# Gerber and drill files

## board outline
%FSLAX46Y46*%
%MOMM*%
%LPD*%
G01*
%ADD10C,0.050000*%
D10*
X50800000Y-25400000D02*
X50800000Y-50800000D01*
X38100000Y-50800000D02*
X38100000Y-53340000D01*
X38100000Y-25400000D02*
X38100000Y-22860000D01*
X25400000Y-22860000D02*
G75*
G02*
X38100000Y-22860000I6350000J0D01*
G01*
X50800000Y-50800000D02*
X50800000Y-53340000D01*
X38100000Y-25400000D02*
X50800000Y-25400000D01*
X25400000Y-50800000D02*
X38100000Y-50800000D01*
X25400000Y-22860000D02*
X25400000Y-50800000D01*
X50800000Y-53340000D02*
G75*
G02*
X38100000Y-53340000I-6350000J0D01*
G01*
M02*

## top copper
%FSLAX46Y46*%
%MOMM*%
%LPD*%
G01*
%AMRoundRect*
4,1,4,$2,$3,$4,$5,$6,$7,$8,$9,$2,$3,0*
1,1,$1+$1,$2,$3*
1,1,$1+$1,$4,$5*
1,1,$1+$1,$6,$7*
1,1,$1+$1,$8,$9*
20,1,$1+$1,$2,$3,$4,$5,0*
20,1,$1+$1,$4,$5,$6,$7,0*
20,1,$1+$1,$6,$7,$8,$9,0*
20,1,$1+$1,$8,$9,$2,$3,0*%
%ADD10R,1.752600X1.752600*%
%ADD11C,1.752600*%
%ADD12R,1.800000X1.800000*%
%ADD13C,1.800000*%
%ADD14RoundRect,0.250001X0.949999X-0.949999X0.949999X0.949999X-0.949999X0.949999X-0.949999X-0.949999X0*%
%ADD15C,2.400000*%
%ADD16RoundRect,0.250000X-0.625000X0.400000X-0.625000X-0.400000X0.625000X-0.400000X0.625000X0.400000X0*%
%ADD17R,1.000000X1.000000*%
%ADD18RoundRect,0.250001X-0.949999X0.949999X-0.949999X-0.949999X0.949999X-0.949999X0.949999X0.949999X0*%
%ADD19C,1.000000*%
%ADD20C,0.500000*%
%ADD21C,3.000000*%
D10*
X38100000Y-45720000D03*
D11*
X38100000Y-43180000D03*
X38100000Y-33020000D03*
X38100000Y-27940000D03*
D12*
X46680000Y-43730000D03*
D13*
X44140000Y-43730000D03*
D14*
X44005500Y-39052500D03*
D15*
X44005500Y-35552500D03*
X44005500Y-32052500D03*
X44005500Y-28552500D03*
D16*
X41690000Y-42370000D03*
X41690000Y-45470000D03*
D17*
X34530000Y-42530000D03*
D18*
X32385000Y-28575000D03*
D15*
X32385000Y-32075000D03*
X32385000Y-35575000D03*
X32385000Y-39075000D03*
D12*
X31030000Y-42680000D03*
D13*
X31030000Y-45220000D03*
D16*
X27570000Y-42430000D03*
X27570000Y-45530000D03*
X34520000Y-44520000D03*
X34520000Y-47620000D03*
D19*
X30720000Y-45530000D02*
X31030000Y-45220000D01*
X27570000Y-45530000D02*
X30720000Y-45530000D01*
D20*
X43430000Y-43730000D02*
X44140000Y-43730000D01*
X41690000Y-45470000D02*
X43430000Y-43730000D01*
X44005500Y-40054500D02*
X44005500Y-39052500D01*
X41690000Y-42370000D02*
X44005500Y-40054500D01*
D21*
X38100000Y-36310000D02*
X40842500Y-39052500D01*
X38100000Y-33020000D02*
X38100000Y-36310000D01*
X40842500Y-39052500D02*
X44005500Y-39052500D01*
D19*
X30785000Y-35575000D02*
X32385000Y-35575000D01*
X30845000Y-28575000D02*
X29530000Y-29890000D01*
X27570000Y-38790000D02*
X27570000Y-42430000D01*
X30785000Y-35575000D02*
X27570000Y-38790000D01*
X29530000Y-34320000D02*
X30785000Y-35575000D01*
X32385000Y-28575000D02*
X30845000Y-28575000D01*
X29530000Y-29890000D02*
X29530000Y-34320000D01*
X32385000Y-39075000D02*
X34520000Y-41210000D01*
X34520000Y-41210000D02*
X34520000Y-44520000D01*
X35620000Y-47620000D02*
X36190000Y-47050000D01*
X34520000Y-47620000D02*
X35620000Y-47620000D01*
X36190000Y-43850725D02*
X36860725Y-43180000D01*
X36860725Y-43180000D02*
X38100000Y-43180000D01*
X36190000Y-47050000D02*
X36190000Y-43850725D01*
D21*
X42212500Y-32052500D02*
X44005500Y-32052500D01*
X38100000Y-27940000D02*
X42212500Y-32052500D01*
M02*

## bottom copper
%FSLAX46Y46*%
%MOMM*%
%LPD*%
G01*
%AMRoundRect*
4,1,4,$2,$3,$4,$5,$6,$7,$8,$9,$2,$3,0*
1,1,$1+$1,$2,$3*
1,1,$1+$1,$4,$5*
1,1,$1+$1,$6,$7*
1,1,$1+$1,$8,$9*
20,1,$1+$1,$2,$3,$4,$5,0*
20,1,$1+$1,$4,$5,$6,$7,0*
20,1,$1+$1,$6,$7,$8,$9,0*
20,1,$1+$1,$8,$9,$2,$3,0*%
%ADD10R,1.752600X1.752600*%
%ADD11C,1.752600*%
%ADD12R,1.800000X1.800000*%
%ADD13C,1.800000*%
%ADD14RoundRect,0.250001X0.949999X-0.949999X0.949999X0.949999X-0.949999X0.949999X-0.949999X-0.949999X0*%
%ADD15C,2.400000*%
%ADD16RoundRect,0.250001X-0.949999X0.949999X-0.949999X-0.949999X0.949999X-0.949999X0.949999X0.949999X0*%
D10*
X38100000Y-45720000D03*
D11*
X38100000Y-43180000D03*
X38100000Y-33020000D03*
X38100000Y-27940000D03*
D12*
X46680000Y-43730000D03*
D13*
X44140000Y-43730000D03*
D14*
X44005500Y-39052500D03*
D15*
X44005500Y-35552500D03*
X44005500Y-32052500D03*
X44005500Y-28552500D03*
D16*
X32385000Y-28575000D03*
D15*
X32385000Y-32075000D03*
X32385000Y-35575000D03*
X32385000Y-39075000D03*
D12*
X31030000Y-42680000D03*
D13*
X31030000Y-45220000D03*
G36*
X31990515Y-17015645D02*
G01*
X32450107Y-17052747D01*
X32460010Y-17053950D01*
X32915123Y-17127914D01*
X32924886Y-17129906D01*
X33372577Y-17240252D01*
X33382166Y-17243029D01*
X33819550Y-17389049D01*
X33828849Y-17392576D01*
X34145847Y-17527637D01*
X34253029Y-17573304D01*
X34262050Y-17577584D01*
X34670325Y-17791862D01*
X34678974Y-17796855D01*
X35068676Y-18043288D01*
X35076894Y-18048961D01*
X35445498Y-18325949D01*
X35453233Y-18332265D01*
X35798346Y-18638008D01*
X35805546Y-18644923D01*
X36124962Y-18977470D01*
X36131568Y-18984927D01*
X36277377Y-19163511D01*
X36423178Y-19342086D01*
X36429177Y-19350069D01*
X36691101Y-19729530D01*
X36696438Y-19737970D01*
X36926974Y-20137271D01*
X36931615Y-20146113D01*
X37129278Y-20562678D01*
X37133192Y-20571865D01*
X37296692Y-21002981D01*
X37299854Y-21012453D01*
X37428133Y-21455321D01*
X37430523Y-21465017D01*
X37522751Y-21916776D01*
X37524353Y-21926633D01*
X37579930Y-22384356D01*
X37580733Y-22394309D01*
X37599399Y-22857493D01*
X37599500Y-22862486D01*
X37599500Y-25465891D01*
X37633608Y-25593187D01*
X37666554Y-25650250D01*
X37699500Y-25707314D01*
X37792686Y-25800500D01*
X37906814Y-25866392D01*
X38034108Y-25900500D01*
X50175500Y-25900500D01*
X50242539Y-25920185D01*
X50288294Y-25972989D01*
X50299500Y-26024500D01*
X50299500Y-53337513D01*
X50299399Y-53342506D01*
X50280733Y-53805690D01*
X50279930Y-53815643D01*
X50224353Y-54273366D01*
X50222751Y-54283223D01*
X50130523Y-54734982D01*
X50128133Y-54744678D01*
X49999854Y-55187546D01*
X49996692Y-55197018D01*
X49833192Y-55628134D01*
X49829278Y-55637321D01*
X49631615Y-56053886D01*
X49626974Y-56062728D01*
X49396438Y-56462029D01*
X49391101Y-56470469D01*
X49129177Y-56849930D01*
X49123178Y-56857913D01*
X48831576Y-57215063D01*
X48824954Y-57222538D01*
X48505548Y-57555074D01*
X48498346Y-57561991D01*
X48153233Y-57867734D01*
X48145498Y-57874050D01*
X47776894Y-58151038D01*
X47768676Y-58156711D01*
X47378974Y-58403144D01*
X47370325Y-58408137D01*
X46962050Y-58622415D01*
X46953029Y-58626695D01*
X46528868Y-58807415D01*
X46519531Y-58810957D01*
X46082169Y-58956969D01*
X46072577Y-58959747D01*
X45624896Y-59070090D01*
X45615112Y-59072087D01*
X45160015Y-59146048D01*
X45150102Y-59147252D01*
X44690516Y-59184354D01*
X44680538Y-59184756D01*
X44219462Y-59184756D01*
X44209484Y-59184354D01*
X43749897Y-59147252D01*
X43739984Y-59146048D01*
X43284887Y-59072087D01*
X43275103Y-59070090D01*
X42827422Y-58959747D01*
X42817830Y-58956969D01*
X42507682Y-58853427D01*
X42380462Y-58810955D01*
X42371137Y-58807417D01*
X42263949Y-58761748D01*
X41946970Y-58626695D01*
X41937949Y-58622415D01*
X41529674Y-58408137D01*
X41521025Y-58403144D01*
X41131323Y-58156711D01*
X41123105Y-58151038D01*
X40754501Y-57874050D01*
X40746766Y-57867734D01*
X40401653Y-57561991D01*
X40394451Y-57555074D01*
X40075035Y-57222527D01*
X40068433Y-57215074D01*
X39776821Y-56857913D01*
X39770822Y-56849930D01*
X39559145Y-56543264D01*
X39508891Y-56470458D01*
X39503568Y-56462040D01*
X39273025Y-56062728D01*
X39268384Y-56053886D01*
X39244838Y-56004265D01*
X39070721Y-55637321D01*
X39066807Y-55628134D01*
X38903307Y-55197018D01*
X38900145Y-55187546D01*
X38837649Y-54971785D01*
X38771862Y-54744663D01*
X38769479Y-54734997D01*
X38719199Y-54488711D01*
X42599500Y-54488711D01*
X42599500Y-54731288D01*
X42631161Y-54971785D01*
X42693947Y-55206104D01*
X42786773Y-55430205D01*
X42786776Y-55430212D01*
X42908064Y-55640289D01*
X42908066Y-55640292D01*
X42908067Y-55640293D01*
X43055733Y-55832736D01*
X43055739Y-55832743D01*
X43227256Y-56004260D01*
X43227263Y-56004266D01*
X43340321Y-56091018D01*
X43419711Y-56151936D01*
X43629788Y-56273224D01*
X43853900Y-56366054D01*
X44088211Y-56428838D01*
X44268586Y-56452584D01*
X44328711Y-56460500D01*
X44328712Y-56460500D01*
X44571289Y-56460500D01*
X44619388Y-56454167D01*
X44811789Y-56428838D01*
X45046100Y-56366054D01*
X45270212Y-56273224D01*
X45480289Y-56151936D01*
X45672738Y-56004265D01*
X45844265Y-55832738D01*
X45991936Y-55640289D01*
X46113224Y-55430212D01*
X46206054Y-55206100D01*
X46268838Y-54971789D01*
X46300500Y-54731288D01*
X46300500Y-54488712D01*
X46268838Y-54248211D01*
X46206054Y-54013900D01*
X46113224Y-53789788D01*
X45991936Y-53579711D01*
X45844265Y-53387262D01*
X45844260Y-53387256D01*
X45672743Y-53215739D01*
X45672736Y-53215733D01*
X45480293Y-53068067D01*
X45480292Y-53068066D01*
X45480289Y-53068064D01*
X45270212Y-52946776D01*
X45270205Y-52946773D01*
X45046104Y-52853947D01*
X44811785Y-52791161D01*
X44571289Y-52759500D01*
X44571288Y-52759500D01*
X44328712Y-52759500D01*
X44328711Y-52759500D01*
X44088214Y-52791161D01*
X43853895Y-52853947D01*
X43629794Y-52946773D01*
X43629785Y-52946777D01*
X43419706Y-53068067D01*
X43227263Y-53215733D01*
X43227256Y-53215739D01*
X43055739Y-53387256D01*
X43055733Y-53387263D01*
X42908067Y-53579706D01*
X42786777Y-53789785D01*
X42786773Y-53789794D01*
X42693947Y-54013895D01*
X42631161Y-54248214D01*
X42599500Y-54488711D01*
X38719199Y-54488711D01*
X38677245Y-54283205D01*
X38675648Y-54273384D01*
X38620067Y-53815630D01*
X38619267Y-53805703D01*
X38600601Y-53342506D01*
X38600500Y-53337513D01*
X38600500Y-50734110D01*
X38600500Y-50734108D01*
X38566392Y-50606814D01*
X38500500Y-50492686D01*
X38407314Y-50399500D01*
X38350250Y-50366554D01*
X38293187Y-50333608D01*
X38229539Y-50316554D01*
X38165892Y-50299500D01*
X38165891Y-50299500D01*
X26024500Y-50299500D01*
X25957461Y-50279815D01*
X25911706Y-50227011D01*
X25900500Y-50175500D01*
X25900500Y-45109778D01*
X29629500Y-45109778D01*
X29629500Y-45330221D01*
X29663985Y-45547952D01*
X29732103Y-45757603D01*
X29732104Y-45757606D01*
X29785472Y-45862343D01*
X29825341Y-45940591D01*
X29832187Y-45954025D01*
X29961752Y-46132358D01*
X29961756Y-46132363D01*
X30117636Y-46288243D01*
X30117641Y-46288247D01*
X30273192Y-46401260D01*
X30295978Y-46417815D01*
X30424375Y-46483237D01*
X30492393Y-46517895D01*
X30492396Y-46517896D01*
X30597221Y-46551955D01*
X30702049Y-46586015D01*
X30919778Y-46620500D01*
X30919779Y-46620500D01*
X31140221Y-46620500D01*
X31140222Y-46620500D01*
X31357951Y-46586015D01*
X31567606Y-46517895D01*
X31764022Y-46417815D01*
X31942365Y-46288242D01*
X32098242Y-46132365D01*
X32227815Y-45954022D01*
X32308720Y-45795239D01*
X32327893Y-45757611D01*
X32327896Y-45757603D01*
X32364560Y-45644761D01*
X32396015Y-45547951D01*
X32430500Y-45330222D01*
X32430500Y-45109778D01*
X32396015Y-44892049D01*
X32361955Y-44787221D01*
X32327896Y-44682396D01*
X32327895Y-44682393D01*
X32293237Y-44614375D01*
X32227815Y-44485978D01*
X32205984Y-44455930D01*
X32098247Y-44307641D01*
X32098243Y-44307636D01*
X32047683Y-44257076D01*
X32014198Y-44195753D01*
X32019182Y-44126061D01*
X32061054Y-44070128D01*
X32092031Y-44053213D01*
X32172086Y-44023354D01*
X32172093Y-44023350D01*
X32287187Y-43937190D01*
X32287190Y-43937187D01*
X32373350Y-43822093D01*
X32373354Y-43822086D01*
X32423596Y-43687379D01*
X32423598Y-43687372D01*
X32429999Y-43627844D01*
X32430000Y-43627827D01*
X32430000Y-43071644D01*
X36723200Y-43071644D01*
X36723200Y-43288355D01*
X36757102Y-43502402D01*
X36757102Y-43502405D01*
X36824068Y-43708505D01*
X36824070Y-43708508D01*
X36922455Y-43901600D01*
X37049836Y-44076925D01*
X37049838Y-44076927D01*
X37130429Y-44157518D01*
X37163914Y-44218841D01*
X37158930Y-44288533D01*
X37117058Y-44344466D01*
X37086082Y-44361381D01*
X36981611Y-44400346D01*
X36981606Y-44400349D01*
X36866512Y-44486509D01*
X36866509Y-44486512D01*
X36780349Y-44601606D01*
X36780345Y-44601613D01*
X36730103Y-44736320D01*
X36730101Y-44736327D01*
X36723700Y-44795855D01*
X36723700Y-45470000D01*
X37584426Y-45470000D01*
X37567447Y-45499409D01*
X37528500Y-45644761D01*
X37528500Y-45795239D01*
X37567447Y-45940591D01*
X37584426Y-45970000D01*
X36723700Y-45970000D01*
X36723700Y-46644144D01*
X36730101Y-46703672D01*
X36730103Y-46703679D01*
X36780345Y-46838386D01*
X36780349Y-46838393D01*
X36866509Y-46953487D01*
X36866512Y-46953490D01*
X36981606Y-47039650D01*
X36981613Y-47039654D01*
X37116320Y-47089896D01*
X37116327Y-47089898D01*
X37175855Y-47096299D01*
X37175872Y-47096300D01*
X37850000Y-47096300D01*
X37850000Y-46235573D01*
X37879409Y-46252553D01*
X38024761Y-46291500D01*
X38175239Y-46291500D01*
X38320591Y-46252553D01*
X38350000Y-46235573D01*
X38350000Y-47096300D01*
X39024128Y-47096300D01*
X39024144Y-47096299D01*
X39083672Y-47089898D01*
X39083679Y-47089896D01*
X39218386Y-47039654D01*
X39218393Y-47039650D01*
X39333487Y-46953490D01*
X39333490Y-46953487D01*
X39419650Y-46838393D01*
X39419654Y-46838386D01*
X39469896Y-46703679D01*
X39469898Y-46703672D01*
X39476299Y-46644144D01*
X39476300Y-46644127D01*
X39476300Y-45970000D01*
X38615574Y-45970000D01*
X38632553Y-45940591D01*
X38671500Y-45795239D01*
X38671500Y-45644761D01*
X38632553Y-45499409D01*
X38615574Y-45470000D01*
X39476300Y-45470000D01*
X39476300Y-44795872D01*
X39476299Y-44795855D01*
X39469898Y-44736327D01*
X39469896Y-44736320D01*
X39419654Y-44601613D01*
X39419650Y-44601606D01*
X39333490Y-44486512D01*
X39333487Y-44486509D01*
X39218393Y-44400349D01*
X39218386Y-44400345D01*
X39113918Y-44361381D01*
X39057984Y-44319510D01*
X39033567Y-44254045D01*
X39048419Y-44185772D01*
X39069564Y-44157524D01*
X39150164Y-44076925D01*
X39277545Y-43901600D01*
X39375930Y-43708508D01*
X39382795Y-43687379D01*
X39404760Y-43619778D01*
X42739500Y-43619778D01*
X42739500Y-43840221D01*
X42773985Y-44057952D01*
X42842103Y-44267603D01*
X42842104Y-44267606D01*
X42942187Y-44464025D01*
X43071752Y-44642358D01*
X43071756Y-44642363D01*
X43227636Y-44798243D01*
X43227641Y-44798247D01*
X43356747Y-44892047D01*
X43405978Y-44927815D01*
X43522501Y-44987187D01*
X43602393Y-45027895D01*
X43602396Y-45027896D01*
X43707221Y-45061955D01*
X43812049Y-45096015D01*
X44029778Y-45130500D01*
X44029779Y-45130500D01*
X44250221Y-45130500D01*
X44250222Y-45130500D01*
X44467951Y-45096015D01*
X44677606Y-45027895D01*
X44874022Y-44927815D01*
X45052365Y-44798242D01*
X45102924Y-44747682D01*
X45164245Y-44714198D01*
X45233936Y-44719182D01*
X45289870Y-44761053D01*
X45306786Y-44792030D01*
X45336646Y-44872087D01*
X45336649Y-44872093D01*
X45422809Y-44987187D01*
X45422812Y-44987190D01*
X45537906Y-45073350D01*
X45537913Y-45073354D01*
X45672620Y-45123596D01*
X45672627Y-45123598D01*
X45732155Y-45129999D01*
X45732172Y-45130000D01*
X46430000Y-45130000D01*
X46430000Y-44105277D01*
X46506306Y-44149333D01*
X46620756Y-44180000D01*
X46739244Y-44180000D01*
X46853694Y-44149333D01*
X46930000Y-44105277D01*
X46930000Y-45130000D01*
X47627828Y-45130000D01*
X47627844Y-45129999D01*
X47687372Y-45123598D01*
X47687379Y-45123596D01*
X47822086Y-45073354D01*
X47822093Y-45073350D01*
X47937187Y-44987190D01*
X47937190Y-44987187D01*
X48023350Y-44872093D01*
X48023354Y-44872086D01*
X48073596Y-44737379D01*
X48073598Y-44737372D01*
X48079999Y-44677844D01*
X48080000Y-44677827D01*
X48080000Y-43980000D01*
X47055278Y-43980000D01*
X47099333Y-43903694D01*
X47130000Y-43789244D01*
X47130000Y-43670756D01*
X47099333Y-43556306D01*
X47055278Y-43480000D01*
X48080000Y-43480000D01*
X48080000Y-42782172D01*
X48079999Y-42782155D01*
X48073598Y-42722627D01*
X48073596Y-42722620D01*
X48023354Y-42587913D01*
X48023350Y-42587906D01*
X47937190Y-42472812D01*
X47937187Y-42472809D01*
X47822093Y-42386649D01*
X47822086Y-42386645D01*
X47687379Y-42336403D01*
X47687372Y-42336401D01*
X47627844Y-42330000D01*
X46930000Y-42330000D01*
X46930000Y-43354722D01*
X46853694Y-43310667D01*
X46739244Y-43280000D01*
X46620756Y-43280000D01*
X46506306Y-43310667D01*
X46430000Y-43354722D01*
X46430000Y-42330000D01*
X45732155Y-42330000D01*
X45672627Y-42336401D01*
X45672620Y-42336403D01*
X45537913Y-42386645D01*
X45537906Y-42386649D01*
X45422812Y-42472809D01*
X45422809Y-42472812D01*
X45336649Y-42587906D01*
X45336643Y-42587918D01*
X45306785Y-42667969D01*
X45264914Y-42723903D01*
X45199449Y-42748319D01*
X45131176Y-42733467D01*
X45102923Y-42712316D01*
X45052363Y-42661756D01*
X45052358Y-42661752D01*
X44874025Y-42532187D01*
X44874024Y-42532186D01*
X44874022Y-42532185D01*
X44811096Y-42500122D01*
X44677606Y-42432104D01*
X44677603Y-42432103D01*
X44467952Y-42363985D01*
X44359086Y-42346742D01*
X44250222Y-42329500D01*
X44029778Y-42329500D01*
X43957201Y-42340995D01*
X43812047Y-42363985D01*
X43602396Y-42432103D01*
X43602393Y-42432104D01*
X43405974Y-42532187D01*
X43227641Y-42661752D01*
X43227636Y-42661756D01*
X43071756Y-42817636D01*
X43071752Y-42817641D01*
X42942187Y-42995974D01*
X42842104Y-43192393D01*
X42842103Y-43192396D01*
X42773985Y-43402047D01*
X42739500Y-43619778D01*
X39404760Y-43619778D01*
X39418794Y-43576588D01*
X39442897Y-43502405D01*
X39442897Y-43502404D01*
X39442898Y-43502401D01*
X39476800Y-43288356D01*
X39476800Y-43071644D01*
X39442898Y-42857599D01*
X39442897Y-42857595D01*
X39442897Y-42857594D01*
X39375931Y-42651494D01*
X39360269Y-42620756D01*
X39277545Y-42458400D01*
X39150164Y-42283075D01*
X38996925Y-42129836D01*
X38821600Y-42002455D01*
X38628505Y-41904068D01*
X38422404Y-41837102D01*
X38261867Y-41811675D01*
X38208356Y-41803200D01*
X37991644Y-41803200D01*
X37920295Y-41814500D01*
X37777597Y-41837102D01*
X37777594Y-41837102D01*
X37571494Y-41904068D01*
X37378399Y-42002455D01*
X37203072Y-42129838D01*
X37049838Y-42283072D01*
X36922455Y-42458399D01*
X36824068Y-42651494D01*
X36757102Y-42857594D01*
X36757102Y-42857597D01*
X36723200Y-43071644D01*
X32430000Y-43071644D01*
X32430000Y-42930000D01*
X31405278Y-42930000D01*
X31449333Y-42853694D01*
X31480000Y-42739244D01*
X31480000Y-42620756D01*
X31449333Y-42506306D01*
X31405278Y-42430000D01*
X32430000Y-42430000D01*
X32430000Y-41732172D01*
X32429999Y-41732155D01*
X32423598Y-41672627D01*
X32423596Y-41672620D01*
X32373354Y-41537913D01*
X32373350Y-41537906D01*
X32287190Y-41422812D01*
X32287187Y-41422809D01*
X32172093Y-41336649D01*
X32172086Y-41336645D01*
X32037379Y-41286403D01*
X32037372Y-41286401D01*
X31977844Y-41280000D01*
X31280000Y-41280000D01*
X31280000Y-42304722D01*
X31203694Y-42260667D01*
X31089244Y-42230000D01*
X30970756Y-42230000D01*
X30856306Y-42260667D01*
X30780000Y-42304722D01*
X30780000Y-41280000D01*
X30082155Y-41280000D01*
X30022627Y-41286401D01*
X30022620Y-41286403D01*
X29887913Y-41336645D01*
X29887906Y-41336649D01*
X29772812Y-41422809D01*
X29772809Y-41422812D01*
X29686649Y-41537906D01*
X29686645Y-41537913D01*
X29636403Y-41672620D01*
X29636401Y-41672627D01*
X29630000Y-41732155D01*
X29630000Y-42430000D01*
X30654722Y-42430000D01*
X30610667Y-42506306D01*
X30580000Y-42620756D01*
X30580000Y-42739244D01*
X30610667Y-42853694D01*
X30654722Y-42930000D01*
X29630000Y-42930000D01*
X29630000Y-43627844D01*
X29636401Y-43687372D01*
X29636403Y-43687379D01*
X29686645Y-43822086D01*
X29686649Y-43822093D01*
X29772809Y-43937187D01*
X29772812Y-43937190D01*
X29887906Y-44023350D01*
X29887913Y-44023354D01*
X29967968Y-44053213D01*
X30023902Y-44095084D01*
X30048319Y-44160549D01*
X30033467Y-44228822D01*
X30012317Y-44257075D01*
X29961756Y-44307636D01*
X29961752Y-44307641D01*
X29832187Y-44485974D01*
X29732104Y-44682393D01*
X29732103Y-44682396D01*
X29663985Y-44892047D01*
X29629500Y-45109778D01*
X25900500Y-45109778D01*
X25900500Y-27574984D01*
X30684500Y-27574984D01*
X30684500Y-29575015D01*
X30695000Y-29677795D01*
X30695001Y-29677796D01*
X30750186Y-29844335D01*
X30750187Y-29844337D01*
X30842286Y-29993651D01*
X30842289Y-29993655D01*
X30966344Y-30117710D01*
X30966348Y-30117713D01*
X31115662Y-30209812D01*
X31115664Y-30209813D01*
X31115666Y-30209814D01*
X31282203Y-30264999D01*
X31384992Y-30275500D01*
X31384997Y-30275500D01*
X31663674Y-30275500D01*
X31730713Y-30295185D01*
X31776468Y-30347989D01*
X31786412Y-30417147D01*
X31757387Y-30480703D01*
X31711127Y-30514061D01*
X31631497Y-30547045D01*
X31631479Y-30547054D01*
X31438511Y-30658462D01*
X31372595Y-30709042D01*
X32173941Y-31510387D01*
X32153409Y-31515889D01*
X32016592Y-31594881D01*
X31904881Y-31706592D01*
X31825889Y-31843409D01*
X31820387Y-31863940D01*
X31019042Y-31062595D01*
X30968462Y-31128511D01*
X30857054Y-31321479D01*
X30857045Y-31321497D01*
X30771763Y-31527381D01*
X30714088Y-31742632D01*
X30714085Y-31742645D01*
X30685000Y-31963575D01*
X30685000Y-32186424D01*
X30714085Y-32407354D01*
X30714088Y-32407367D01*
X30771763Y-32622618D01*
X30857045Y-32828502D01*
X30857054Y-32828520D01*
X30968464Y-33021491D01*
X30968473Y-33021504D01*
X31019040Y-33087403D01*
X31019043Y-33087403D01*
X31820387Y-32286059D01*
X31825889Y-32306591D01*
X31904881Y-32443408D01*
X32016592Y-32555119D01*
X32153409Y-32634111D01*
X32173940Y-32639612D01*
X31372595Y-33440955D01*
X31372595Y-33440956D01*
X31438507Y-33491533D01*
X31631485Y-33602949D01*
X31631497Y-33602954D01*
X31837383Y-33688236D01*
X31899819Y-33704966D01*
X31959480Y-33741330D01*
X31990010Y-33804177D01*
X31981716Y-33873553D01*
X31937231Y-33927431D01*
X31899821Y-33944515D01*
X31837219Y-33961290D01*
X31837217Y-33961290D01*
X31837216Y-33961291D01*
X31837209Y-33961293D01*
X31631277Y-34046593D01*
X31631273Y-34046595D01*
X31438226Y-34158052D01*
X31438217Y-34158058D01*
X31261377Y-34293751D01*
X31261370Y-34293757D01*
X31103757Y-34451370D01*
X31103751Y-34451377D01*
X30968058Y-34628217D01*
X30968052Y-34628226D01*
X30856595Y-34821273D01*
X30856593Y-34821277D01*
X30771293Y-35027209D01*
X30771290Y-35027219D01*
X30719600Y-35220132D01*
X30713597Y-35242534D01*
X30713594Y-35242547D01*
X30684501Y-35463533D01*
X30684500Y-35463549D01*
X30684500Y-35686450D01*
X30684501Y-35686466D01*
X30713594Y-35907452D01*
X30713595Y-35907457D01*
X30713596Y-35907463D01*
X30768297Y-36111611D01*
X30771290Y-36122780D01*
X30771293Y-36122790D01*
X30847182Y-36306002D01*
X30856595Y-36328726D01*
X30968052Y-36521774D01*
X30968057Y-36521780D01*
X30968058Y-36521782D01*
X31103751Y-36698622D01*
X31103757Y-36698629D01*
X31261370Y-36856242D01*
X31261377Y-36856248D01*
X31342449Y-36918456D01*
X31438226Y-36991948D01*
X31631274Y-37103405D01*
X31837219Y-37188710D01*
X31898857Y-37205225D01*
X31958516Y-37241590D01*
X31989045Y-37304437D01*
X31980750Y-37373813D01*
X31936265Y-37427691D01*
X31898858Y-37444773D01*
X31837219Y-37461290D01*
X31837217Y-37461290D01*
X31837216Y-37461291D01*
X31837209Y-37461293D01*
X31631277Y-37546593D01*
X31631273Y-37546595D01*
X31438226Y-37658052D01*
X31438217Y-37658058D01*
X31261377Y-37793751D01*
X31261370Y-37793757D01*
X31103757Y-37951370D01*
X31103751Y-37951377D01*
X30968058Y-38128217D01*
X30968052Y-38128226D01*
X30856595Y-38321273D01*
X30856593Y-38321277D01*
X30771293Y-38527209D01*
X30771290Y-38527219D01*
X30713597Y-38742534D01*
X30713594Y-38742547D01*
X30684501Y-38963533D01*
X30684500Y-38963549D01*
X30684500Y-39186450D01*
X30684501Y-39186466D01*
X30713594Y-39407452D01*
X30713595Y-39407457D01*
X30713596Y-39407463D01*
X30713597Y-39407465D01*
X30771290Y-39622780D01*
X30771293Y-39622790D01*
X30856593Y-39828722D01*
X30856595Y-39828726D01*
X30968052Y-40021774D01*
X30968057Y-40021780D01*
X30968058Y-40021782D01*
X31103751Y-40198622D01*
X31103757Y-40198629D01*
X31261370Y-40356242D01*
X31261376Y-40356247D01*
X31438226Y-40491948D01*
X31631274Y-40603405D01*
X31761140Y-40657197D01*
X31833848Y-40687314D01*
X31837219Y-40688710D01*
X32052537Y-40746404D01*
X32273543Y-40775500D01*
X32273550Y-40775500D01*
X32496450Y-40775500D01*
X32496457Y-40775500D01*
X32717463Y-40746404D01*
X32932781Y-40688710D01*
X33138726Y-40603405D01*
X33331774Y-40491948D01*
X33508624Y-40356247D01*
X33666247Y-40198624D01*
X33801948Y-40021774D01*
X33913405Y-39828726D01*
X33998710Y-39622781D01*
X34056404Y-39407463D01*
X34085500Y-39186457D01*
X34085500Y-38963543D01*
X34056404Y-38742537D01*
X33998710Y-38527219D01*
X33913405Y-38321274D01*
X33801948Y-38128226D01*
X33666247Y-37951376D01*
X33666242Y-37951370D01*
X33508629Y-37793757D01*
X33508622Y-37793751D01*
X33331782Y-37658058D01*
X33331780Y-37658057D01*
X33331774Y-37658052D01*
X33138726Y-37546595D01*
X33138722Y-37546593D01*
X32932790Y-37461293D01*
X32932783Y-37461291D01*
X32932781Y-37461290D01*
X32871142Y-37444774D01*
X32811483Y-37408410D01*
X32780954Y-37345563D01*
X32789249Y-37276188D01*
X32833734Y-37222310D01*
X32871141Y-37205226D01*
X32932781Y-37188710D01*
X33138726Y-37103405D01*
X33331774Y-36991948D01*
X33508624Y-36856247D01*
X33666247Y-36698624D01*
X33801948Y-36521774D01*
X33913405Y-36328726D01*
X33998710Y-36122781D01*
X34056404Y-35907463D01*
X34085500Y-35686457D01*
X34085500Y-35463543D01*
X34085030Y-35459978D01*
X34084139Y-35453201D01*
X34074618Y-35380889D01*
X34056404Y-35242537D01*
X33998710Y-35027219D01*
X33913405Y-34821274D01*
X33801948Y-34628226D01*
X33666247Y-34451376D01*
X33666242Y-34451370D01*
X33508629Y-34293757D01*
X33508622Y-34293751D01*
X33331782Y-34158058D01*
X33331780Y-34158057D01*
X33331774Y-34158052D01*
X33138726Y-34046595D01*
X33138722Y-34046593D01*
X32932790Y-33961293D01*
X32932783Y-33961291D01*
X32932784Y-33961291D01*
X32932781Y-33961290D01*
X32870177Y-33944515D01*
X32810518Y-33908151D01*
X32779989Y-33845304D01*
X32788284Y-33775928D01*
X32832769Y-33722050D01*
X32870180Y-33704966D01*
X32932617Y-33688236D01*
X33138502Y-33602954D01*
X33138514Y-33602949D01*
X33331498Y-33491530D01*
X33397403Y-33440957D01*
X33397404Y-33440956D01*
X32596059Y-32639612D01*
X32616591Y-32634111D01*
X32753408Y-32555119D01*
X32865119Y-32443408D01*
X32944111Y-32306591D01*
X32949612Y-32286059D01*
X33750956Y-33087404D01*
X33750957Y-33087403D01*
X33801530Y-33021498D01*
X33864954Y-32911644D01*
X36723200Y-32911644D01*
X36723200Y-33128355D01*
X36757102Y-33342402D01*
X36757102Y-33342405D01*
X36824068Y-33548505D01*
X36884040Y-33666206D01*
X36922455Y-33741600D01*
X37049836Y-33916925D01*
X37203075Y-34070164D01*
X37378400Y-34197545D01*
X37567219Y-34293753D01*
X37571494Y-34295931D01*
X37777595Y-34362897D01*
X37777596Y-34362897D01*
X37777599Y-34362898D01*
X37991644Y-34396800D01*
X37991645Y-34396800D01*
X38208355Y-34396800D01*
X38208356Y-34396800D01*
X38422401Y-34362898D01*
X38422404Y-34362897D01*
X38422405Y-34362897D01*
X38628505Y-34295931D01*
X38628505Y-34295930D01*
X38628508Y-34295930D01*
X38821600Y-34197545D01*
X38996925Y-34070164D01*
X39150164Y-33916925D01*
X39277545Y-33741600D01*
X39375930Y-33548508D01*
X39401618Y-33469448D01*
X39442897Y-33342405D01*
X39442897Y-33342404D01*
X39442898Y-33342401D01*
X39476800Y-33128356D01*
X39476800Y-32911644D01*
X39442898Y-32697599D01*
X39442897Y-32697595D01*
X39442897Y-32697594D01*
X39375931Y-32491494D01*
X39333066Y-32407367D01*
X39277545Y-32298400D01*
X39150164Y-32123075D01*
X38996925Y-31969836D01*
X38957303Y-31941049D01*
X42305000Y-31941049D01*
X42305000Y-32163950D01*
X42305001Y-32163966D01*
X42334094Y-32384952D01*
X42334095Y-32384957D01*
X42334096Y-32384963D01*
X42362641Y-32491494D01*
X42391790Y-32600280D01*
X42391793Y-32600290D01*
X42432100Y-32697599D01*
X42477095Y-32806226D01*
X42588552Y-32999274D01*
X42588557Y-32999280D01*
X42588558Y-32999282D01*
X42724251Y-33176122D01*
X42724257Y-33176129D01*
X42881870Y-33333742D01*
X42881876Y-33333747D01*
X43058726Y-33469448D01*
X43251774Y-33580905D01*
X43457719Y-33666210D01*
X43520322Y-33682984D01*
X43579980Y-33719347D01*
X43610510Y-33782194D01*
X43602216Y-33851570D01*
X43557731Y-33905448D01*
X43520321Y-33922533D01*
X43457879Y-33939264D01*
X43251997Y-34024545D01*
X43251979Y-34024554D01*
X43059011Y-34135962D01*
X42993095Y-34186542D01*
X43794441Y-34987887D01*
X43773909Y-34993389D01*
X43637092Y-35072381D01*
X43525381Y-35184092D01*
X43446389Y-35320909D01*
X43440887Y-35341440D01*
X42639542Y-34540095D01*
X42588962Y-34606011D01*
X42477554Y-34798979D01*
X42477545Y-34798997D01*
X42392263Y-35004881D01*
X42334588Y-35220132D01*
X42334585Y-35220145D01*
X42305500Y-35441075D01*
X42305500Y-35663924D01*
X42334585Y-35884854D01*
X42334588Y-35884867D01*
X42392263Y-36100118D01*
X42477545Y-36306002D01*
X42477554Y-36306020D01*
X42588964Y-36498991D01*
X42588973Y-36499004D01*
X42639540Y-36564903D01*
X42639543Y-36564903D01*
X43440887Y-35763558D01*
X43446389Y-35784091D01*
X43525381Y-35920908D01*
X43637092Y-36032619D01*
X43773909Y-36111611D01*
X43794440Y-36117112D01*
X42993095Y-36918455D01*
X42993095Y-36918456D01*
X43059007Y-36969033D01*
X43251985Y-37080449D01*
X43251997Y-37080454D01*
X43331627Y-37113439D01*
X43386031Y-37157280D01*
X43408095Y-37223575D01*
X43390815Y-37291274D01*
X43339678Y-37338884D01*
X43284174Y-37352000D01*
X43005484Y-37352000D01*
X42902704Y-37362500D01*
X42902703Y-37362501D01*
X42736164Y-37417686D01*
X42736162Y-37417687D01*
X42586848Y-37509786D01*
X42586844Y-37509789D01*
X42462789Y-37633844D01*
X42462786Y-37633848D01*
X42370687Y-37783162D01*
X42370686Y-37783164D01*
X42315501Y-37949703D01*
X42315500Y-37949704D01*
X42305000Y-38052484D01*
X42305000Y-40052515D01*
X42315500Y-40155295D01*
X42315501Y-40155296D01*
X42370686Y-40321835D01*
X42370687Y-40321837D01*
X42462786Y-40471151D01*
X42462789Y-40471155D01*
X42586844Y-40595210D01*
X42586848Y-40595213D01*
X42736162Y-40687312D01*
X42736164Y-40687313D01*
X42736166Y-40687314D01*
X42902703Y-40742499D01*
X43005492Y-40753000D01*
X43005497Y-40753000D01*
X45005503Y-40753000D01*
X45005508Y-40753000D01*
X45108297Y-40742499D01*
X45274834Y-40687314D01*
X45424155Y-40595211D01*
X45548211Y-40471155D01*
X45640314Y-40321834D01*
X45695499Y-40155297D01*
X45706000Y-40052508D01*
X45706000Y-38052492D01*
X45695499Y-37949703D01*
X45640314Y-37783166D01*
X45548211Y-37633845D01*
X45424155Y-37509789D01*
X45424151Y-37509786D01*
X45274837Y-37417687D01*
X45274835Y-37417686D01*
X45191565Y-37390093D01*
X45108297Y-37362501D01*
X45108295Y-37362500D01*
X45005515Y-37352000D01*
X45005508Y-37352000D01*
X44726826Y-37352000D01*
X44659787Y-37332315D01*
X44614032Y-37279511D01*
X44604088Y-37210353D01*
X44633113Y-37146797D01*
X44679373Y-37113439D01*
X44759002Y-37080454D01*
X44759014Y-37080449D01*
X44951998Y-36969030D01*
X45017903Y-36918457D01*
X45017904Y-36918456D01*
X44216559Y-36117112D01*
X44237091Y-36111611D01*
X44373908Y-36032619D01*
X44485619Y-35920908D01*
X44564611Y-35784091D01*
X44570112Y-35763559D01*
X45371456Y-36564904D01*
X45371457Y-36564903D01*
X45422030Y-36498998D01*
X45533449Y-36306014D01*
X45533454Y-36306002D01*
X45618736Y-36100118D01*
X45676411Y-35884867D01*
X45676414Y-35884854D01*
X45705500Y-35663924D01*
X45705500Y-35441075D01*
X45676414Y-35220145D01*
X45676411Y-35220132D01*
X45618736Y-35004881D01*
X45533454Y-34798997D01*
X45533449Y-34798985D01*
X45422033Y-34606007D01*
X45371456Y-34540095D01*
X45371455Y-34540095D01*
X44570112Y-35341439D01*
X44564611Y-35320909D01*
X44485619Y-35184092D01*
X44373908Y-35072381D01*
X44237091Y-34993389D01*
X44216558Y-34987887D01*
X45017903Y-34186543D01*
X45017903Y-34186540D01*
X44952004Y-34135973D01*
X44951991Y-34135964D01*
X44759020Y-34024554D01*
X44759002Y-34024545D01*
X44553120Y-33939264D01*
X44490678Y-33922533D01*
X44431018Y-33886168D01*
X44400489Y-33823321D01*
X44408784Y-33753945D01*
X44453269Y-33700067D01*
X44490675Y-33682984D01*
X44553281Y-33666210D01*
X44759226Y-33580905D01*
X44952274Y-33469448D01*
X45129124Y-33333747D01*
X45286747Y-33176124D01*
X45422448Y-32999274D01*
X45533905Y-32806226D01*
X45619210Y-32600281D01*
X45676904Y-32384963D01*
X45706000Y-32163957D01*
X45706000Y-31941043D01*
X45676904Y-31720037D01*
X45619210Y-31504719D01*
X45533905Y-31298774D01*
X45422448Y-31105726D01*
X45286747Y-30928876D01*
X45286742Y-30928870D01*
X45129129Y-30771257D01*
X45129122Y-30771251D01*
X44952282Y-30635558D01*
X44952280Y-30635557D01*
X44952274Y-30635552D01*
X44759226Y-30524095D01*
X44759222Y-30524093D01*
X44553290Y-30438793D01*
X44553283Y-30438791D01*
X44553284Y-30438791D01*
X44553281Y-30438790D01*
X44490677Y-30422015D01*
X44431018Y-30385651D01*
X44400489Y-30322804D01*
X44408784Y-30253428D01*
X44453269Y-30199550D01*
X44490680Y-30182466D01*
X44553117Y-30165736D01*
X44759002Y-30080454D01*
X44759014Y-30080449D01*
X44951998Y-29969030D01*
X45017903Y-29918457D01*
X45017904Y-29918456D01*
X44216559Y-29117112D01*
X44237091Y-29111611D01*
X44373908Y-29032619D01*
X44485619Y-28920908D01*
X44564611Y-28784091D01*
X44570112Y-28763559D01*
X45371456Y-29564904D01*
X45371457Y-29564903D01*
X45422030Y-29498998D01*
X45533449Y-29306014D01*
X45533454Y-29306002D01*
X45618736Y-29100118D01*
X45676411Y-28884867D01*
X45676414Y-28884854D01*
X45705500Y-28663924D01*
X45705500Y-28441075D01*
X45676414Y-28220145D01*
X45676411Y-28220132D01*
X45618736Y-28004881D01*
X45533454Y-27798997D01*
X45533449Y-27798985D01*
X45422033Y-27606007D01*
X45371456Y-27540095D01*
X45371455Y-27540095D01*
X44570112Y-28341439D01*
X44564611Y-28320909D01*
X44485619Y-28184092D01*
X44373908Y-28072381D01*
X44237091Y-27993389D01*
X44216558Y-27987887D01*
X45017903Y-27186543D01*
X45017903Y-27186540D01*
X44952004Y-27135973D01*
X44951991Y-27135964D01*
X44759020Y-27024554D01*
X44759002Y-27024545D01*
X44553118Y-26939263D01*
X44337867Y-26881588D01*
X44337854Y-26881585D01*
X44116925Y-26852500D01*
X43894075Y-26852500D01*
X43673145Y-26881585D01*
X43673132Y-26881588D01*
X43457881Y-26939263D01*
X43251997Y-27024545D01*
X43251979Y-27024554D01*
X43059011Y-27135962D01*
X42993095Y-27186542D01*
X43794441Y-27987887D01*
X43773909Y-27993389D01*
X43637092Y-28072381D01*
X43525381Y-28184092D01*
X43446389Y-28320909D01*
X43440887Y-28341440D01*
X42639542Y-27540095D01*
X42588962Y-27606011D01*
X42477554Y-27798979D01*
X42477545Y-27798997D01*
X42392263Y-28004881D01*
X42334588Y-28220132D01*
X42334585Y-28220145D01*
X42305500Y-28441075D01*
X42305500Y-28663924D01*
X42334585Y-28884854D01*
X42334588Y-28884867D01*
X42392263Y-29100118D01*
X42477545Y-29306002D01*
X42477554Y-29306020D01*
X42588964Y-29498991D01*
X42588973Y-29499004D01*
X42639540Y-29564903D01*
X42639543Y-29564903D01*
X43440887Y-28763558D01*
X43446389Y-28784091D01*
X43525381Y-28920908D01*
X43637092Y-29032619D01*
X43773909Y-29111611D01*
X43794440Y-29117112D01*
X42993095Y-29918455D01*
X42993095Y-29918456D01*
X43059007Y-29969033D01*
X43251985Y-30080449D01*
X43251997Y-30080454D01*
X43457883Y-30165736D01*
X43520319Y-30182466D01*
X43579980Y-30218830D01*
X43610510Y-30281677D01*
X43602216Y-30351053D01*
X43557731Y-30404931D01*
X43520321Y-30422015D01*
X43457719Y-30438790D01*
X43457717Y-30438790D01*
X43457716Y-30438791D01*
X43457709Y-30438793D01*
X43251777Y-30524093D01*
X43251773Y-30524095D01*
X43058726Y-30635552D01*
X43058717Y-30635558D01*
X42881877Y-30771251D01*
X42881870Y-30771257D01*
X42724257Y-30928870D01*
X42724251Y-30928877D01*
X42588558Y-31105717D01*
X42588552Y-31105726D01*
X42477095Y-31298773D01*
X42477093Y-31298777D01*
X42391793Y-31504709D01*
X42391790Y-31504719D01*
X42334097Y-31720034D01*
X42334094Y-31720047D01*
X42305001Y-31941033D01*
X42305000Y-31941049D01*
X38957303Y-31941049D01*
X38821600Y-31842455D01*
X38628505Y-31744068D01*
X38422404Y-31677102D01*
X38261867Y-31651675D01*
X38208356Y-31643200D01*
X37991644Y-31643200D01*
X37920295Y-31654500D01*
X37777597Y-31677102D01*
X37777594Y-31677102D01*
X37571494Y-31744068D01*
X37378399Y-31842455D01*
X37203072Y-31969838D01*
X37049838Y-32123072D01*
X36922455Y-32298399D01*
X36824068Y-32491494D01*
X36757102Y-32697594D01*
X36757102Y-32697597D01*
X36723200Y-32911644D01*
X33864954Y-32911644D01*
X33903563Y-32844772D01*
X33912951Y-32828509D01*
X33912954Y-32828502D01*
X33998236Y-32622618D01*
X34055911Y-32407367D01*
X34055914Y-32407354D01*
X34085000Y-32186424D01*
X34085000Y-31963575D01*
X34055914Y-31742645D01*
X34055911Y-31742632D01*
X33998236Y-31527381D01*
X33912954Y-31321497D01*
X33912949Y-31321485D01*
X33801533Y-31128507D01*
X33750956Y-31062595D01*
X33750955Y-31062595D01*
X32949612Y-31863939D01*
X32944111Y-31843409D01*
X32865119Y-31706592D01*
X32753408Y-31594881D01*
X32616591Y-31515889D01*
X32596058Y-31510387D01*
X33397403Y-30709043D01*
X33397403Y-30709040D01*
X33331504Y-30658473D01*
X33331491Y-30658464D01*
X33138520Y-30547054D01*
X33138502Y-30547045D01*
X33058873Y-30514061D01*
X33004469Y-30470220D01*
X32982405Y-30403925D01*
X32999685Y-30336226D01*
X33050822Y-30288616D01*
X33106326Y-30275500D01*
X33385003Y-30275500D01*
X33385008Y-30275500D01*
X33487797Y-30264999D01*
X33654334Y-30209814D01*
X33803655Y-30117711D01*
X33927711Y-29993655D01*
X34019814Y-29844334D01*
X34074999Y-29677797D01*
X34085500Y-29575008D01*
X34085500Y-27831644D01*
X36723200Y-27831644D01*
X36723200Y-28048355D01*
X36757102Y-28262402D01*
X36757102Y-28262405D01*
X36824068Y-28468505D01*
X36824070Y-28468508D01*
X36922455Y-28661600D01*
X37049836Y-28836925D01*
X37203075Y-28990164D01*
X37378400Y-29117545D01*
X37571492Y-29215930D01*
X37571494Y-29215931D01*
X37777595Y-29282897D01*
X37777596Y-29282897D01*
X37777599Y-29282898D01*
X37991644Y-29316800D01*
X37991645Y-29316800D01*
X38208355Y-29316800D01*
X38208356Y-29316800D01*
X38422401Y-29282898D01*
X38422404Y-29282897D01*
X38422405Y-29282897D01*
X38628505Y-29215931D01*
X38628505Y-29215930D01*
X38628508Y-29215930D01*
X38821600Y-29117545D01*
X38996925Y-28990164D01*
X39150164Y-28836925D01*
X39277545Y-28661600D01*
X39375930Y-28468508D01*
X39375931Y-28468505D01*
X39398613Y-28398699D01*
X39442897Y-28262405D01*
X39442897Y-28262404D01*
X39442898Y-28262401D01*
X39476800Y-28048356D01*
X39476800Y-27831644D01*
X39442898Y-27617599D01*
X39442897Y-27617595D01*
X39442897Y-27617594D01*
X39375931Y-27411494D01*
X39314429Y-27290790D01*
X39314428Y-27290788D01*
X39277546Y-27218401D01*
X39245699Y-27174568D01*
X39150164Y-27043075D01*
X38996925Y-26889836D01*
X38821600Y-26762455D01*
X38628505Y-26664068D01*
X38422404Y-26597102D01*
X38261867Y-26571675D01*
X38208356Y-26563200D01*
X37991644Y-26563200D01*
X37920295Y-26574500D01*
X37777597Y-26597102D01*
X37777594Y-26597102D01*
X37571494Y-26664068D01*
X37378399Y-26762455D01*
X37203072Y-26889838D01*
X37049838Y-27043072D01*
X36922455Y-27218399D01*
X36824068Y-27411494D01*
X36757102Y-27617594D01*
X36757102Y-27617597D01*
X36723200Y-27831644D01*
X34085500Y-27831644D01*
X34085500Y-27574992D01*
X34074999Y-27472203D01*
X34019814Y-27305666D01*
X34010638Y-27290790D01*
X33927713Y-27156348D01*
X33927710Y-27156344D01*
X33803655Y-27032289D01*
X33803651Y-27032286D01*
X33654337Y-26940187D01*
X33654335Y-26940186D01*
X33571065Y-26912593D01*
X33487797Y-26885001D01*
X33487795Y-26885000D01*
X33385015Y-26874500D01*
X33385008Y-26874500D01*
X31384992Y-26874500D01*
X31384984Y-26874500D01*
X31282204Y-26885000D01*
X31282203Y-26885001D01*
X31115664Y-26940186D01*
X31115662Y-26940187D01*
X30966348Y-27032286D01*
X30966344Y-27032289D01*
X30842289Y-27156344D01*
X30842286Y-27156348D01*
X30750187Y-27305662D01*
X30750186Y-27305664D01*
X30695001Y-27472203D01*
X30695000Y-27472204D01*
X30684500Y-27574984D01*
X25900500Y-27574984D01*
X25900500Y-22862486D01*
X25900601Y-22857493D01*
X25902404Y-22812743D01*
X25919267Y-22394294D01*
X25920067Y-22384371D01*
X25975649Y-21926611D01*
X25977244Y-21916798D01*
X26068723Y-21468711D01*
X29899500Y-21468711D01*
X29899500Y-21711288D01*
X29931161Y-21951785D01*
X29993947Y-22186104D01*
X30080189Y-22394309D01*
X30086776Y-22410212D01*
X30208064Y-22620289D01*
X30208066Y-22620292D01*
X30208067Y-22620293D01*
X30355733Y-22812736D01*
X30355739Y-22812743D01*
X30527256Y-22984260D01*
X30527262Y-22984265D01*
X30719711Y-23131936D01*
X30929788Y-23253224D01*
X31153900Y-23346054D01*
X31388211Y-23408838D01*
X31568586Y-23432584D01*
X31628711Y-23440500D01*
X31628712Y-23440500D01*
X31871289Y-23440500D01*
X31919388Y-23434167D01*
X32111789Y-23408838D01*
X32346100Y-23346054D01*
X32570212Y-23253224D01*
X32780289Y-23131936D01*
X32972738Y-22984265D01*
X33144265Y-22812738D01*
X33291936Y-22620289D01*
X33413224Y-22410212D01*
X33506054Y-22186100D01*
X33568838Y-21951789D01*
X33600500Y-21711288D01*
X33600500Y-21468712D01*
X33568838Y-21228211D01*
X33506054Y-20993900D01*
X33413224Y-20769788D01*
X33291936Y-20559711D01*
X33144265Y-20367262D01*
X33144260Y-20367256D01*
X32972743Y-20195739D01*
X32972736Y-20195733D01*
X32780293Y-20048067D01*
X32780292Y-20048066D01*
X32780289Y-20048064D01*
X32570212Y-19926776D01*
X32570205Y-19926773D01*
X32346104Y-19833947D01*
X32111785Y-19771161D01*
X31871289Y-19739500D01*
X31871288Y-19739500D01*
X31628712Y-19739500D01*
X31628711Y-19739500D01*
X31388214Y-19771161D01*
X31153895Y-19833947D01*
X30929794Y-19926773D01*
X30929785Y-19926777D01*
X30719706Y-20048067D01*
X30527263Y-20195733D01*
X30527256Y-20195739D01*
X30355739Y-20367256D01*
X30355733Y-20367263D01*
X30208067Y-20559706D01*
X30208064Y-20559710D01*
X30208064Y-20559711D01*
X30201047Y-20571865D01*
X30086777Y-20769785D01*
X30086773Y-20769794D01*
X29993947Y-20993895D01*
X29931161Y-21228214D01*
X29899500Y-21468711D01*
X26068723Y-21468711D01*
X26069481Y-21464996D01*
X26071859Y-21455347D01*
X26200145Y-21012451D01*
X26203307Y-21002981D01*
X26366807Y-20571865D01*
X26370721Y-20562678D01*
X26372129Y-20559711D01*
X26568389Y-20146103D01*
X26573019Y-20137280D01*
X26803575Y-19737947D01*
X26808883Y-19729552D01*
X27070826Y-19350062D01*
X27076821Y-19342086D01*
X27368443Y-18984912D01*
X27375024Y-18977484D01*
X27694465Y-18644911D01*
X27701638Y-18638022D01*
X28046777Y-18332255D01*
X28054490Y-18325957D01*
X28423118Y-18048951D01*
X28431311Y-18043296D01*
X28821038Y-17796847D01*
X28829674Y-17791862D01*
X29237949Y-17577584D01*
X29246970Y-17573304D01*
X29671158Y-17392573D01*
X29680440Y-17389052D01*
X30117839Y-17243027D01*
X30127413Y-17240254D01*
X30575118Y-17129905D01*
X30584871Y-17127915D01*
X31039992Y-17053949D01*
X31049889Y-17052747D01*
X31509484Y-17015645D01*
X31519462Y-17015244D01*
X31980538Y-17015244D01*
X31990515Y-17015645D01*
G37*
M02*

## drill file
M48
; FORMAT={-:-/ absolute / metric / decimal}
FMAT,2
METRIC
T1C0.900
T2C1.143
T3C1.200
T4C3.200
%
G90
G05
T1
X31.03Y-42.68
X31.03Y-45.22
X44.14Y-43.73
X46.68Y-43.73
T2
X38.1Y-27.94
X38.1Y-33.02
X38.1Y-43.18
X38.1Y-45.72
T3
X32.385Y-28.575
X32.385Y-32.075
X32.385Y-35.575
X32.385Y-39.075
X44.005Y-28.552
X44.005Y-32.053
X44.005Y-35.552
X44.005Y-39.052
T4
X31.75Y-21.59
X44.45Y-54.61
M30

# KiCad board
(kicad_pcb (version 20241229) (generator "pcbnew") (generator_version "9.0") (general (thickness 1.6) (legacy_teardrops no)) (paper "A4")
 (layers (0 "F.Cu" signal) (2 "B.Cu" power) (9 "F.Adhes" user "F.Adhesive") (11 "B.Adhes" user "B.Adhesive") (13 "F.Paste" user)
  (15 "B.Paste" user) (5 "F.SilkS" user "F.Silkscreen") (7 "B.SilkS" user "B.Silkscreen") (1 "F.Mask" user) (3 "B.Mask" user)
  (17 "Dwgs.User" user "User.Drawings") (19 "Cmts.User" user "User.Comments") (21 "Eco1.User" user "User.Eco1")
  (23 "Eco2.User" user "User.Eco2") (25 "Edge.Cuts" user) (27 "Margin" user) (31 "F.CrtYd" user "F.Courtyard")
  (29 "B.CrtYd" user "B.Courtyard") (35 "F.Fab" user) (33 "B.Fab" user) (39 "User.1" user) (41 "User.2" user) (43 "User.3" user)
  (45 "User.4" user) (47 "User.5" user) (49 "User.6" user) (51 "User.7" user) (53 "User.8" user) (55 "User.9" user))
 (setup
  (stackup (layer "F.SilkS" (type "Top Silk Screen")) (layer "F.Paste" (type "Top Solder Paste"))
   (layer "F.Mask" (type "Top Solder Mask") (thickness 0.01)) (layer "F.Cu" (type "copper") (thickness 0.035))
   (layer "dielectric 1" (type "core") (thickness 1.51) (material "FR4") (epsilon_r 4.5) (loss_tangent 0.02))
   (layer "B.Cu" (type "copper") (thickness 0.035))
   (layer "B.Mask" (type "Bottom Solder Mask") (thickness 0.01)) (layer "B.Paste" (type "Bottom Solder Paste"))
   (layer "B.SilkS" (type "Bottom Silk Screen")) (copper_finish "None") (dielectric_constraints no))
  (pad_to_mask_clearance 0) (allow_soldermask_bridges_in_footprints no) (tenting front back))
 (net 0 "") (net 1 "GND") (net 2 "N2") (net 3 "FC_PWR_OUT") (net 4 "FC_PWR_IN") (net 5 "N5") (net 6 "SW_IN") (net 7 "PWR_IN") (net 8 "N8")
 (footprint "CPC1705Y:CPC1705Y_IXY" (layer "F.Cu") (at 38.1 45.72 90)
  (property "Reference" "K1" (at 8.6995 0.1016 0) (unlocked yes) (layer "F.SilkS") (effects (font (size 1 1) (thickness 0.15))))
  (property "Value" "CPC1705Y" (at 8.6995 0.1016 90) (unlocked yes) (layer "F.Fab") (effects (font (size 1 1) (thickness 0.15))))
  (pad "1" thru_hole rect (at 0 0 90) (size 1.7526 1.7526) (drill 1.143) (layers "*.Cu" "*.Mask") (remove_unused_layers no) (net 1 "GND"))
  (pad "2" thru_hole circle (at 2.54 0 90) (size 1.7526 1.7526) (drill 1.143) (layers "*.Cu" "*.Mask") (remove_unused_layers no)
   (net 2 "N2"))
  (pad "3" thru_hole circle (at 12.7 0 90) (size 1.7526 1.7526) (drill 1.143) (layers "*.Cu" "*.Mask") (remove_unused_layers no)
   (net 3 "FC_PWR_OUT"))
  (pad "4" thru_hole circle (at 17.78 0 90) (size 1.7526 1.7526) (drill 1.143) (layers "*.Cu" "*.Mask") (remove_unused_layers no)
   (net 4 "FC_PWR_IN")))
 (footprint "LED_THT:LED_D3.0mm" (layer "F.Cu") (at 46.68 43.73 180)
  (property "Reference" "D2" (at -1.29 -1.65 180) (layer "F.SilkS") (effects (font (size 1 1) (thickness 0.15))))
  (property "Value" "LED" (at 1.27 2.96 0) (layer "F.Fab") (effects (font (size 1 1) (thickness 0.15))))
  (pad "1" thru_hole rect (at 0 0 180) (size 1.8 1.8) (drill 0.9) (layers "*.Cu" "*.Mask") (remove_unused_layers no) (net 1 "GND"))
  (pad "2" thru_hole circle (at 2.54 0 180) (size 1.8 1.8) (drill 0.9) (layers "*.Cu" "*.Mask") (remove_unused_layers no) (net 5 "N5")))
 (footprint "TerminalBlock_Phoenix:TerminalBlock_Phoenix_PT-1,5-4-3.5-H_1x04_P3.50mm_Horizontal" (layer "F.Cu") (at 44.0055 39.0525 90)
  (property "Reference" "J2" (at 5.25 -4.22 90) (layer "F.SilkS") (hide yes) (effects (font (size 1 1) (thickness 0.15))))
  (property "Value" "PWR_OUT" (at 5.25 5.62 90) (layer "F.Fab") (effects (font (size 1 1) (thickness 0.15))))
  (pad "1" thru_hole roundrect (at 0 0 90) (size 2.4 2.4) (drill 1.2) (layers "*.Cu" "*.Mask") (remove_unused_layers no)
   (roundrect_rratio 0.104167) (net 3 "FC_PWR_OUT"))
  (pad "2" thru_hole circle (at 3.5 0 90) (size 2.4 2.4) (drill 1.2) (layers "*.Cu" "*.Mask") (remove_unused_layers no) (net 1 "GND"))
  (pad "3" thru_hole circle (at 7 0 90) (size 2.4 2.4) (drill 1.2) (layers "*.Cu" "*.Mask") (remove_unused_layers no) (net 4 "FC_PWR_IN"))
  (pad "4" thru_hole circle (at 10.5 0 90) (size 2.4 2.4) (drill 1.2) (layers "*.Cu" "*.Mask") (remove_unused_layers no) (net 1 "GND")))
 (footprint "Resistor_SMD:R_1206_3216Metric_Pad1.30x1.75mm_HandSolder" (layer "F.Cu") (at 41.69 43.92 -90)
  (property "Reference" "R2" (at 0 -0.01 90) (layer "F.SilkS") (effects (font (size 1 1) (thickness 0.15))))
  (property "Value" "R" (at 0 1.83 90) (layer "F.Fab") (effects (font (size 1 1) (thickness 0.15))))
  (pad "1" smd roundrect (at -1.55 0 270) (size 1.3 1.75) (layers "F.Cu" "F.Mask" "F.Paste") (roundrect_rratio 0.192308)
   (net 3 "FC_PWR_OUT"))
  (pad "2" smd roundrect (at 1.55 0 270) (size 1.3 1.75) (layers "F.Cu" "F.Mask" "F.Paste") (roundrect_rratio 0.192308) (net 5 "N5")))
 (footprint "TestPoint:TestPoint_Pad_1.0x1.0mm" (layer "F.Cu") (at 34.53 42.53)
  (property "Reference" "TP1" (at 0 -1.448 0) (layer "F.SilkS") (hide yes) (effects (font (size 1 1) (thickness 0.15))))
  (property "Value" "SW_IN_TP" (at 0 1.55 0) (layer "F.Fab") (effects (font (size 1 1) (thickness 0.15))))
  (pad "1" smd rect (at 0 0) (size 1 1) (layers "F.Cu" "F.Mask") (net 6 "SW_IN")))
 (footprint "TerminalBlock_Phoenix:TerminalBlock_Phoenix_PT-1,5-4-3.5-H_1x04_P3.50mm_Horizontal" (layer "F.Cu") (at 32.385 28.575 -90)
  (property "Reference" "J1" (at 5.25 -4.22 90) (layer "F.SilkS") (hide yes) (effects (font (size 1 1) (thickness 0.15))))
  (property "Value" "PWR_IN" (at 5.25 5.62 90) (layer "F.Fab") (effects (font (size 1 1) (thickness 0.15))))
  (pad "1" thru_hole roundrect (at 0 0 270) (size 2.4 2.4) (drill 1.2) (layers "*.Cu" "*.Mask") (remove_unused_layers no)
   (roundrect_rratio 0.104167) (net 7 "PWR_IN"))
  (pad "2" thru_hole circle (at 3.5 0 270) (size 2.4 2.4) (drill 1.2) (layers "*.Cu" "*.Mask") (remove_unused_layers no) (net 1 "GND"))
  (pad "3" thru_hole circle (at 7 0 270) (size 2.4 2.4) (drill 1.2) (layers "*.Cu" "*.Mask") (remove_unused_layers no) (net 7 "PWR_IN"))
  (pad "4" thru_hole circle (at 10.5 0 270) (size 2.4 2.4) (drill 1.2) (layers "*.Cu" "*.Mask") (remove_unused_layers no) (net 6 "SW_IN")))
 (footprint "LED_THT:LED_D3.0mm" (layer "F.Cu") (at 31.03 42.68 -90)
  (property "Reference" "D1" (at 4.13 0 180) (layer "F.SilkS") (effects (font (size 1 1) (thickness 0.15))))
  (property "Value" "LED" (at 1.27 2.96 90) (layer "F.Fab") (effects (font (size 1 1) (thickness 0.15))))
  (pad "1" thru_hole rect (at 0 0 270) (size 1.8 1.8) (drill 0.9) (layers "*.Cu" "*.Mask") (remove_unused_layers no) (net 1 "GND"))
  (pad "2" thru_hole circle (at 2.54 0 270) (size 1.8 1.8) (drill 0.9) (layers "*.Cu" "*.Mask") (remove_unused_layers no) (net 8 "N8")))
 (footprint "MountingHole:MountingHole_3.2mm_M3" (layer "F.Cu") (at 44.45 54.61)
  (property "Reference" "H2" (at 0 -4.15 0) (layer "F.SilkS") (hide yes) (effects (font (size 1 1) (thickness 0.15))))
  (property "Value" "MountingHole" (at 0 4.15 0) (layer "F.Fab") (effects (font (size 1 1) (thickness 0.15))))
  (pad "" np_thru_hole circle (at 0 0) (size 3.2 3.2) (drill 3.2) (layers "*.Cu" "*.Mask")))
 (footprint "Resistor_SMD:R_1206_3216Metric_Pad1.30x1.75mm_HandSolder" (layer "F.Cu") (at 27.57 43.98 -90)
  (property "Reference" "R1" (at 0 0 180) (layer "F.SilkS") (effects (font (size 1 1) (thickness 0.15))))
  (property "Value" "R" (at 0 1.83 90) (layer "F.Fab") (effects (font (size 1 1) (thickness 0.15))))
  (pad "1" smd roundrect (at -1.55 0 270) (size 1.3 1.75) (layers "F.Cu" "F.Mask" "F.Paste") (roundrect_rratio 0.192308) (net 7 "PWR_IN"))
  (pad "2" smd roundrect (at 1.55 0 270) (size 1.3 1.75) (layers "F.Cu" "F.Mask" "F.Paste") (roundrect_rratio 0.192308) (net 8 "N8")))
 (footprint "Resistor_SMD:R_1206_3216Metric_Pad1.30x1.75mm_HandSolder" (layer "F.Cu") (at 34.52 46.07 -90)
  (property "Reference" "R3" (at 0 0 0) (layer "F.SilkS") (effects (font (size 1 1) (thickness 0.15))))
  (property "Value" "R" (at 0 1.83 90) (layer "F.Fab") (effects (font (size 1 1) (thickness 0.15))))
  (pad "1" smd roundrect (at -1.55 0 270) (size 1.3 1.75) (layers "F.Cu" "F.Mask" "F.Paste") (roundrect_rratio 0.192308) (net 6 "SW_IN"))
  (pad "2" smd roundrect (at 1.55 0 270) (size 1.3 1.75) (layers "F.Cu" "F.Mask" "F.Paste") (roundrect_rratio 0.192308) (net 2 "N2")))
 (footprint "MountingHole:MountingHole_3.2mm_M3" (layer "F.Cu") (at 31.75 21.59)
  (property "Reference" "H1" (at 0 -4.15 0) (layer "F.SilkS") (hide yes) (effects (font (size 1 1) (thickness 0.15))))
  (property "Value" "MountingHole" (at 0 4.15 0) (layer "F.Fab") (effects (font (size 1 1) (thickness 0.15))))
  (pad "" np_thru_hole circle (at 0 0) (size 3.2 3.2) (drill 3.2) (layers "*.Cu" "*.Mask")))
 (gr_line (start 50.8 25.4) (end 50.8 50.8) (stroke (width 0.05) (type solid)) (layer "Edge.Cuts"))
 (gr_line (start 38.1 50.8) (end 38.1 53.34) (stroke (width 0.05) (type solid)) (layer "Edge.Cuts"))
 (gr_line (start 38.1 25.4) (end 38.1 22.86) (stroke (width 0.05) (type solid)) (layer "Edge.Cuts"))
 (gr_arc (start 25.4 22.86) (mid 31.75 16.51) (end 38.1 22.86) (stroke (width 0.05) (type solid)) (layer "Edge.Cuts"))
 (gr_line (start 50.8 50.8) (end 50.8 53.34) (stroke (width 0.05) (type solid)) (layer "Edge.Cuts"))
 (gr_line (start 38.1 25.4) (end 50.8 25.4) (stroke (width 0.05) (type solid)) (layer "Edge.Cuts"))
 (gr_line (start 25.4 50.8) (end 38.1 50.8) (stroke (width 0.05) (type solid)) (layer "Edge.Cuts"))
 (gr_line (start 25.4 22.86) (end 25.4 50.8) (stroke (width 0.05) (type solid)) (layer "Edge.Cuts"))
 (gr_arc (start 50.8 53.34) (mid 44.45 59.69) (end 38.1 53.34) (stroke (width 0.05) (type solid)) (layer "Edge.Cuts"))
 (segment (start 30.72 45.53) (end 31.03 45.22) (width 1) (layer "F.Cu") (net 8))
 (segment (start 27.57 45.53) (end 30.72 45.53) (width 1) (layer "F.Cu") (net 8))
 (segment (start 43.43 43.73) (end 44.14 43.73) (width 0.5) (layer "F.Cu") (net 5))
 (segment (start 41.69 45.47) (end 43.43 43.73) (width 0.5) (layer "F.Cu") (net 5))
 (segment (start 44.0055 40.0545) (end 44.0055 39.0525) (width 0.5) (layer "F.Cu") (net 3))
 (segment (start 41.69 42.37) (end 44.0055 40.0545) (width 0.5) (layer "F.Cu") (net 3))
 (segment (start 38.1 36.31) (end 40.8425 39.0525) (width 3) (layer "F.Cu") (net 3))
 (segment (start 38.1 33.02) (end 38.1 36.31) (width 3) (layer "F.Cu") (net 3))
 (segment (start 40.8425 39.0525) (end 44.0055 39.0525) (width 3) (layer "F.Cu") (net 3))
 (segment (start 30.785 35.575) (end 32.385 35.575) (width 1) (layer "F.Cu") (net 7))
 (segment (start 30.845 28.575) (end 29.53 29.89) (width 1) (layer "F.Cu") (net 7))
 (segment (start 27.57 38.79) (end 27.57 42.43) (width 1) (layer "F.Cu") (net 7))
 (segment (start 30.785 35.575) (end 27.57 38.79) (width 1) (layer "F.Cu") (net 7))
 (segment (start 29.53 34.32) (end 30.785 35.575) (width 1) (layer "F.Cu") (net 7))
 (segment (start 32.385 28.575) (end 30.845 28.575) (width 1) (layer "F.Cu") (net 7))
 (segment (start 29.53 29.89) (end 29.53 34.32) (width 1) (layer "F.Cu") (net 7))
 (segment (start 32.385 39.075) (end 34.52 41.21) (width 1) (layer "F.Cu") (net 6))
 (segment (start 34.52 41.21) (end 34.52 44.52) (width 1) (layer "F.Cu") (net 6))
 (segment (start 35.62 47.62) (end 36.19 47.05) (width 1) (layer "F.Cu") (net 2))
 (segment (start 34.52 47.62) (end 35.62 47.62) (width 1) (layer "F.Cu") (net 2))
 (segment (start 36.19 43.850725) (end 36.860725 43.18) (width 1) (layer "F.Cu") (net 2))
 (segment (start 36.860725 43.18) (end 38.1 43.18) (width 1) (layer "F.Cu") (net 2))
 (segment (start 36.19 47.05) (end 36.19 43.850725) (width 1) (layer "F.Cu") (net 2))
 (segment (start 42.2125 32.0525) (end 44.0055 32.0525) (width 3) (layer "F.Cu") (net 4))
 (segment (start 38.1 27.94) (end 42.2125 32.0525) (width 3) (layer "F.Cu") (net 4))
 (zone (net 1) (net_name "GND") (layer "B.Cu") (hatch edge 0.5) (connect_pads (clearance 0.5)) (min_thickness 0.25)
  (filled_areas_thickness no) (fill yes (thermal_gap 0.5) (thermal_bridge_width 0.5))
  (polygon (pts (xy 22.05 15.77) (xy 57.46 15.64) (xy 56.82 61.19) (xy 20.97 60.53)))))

